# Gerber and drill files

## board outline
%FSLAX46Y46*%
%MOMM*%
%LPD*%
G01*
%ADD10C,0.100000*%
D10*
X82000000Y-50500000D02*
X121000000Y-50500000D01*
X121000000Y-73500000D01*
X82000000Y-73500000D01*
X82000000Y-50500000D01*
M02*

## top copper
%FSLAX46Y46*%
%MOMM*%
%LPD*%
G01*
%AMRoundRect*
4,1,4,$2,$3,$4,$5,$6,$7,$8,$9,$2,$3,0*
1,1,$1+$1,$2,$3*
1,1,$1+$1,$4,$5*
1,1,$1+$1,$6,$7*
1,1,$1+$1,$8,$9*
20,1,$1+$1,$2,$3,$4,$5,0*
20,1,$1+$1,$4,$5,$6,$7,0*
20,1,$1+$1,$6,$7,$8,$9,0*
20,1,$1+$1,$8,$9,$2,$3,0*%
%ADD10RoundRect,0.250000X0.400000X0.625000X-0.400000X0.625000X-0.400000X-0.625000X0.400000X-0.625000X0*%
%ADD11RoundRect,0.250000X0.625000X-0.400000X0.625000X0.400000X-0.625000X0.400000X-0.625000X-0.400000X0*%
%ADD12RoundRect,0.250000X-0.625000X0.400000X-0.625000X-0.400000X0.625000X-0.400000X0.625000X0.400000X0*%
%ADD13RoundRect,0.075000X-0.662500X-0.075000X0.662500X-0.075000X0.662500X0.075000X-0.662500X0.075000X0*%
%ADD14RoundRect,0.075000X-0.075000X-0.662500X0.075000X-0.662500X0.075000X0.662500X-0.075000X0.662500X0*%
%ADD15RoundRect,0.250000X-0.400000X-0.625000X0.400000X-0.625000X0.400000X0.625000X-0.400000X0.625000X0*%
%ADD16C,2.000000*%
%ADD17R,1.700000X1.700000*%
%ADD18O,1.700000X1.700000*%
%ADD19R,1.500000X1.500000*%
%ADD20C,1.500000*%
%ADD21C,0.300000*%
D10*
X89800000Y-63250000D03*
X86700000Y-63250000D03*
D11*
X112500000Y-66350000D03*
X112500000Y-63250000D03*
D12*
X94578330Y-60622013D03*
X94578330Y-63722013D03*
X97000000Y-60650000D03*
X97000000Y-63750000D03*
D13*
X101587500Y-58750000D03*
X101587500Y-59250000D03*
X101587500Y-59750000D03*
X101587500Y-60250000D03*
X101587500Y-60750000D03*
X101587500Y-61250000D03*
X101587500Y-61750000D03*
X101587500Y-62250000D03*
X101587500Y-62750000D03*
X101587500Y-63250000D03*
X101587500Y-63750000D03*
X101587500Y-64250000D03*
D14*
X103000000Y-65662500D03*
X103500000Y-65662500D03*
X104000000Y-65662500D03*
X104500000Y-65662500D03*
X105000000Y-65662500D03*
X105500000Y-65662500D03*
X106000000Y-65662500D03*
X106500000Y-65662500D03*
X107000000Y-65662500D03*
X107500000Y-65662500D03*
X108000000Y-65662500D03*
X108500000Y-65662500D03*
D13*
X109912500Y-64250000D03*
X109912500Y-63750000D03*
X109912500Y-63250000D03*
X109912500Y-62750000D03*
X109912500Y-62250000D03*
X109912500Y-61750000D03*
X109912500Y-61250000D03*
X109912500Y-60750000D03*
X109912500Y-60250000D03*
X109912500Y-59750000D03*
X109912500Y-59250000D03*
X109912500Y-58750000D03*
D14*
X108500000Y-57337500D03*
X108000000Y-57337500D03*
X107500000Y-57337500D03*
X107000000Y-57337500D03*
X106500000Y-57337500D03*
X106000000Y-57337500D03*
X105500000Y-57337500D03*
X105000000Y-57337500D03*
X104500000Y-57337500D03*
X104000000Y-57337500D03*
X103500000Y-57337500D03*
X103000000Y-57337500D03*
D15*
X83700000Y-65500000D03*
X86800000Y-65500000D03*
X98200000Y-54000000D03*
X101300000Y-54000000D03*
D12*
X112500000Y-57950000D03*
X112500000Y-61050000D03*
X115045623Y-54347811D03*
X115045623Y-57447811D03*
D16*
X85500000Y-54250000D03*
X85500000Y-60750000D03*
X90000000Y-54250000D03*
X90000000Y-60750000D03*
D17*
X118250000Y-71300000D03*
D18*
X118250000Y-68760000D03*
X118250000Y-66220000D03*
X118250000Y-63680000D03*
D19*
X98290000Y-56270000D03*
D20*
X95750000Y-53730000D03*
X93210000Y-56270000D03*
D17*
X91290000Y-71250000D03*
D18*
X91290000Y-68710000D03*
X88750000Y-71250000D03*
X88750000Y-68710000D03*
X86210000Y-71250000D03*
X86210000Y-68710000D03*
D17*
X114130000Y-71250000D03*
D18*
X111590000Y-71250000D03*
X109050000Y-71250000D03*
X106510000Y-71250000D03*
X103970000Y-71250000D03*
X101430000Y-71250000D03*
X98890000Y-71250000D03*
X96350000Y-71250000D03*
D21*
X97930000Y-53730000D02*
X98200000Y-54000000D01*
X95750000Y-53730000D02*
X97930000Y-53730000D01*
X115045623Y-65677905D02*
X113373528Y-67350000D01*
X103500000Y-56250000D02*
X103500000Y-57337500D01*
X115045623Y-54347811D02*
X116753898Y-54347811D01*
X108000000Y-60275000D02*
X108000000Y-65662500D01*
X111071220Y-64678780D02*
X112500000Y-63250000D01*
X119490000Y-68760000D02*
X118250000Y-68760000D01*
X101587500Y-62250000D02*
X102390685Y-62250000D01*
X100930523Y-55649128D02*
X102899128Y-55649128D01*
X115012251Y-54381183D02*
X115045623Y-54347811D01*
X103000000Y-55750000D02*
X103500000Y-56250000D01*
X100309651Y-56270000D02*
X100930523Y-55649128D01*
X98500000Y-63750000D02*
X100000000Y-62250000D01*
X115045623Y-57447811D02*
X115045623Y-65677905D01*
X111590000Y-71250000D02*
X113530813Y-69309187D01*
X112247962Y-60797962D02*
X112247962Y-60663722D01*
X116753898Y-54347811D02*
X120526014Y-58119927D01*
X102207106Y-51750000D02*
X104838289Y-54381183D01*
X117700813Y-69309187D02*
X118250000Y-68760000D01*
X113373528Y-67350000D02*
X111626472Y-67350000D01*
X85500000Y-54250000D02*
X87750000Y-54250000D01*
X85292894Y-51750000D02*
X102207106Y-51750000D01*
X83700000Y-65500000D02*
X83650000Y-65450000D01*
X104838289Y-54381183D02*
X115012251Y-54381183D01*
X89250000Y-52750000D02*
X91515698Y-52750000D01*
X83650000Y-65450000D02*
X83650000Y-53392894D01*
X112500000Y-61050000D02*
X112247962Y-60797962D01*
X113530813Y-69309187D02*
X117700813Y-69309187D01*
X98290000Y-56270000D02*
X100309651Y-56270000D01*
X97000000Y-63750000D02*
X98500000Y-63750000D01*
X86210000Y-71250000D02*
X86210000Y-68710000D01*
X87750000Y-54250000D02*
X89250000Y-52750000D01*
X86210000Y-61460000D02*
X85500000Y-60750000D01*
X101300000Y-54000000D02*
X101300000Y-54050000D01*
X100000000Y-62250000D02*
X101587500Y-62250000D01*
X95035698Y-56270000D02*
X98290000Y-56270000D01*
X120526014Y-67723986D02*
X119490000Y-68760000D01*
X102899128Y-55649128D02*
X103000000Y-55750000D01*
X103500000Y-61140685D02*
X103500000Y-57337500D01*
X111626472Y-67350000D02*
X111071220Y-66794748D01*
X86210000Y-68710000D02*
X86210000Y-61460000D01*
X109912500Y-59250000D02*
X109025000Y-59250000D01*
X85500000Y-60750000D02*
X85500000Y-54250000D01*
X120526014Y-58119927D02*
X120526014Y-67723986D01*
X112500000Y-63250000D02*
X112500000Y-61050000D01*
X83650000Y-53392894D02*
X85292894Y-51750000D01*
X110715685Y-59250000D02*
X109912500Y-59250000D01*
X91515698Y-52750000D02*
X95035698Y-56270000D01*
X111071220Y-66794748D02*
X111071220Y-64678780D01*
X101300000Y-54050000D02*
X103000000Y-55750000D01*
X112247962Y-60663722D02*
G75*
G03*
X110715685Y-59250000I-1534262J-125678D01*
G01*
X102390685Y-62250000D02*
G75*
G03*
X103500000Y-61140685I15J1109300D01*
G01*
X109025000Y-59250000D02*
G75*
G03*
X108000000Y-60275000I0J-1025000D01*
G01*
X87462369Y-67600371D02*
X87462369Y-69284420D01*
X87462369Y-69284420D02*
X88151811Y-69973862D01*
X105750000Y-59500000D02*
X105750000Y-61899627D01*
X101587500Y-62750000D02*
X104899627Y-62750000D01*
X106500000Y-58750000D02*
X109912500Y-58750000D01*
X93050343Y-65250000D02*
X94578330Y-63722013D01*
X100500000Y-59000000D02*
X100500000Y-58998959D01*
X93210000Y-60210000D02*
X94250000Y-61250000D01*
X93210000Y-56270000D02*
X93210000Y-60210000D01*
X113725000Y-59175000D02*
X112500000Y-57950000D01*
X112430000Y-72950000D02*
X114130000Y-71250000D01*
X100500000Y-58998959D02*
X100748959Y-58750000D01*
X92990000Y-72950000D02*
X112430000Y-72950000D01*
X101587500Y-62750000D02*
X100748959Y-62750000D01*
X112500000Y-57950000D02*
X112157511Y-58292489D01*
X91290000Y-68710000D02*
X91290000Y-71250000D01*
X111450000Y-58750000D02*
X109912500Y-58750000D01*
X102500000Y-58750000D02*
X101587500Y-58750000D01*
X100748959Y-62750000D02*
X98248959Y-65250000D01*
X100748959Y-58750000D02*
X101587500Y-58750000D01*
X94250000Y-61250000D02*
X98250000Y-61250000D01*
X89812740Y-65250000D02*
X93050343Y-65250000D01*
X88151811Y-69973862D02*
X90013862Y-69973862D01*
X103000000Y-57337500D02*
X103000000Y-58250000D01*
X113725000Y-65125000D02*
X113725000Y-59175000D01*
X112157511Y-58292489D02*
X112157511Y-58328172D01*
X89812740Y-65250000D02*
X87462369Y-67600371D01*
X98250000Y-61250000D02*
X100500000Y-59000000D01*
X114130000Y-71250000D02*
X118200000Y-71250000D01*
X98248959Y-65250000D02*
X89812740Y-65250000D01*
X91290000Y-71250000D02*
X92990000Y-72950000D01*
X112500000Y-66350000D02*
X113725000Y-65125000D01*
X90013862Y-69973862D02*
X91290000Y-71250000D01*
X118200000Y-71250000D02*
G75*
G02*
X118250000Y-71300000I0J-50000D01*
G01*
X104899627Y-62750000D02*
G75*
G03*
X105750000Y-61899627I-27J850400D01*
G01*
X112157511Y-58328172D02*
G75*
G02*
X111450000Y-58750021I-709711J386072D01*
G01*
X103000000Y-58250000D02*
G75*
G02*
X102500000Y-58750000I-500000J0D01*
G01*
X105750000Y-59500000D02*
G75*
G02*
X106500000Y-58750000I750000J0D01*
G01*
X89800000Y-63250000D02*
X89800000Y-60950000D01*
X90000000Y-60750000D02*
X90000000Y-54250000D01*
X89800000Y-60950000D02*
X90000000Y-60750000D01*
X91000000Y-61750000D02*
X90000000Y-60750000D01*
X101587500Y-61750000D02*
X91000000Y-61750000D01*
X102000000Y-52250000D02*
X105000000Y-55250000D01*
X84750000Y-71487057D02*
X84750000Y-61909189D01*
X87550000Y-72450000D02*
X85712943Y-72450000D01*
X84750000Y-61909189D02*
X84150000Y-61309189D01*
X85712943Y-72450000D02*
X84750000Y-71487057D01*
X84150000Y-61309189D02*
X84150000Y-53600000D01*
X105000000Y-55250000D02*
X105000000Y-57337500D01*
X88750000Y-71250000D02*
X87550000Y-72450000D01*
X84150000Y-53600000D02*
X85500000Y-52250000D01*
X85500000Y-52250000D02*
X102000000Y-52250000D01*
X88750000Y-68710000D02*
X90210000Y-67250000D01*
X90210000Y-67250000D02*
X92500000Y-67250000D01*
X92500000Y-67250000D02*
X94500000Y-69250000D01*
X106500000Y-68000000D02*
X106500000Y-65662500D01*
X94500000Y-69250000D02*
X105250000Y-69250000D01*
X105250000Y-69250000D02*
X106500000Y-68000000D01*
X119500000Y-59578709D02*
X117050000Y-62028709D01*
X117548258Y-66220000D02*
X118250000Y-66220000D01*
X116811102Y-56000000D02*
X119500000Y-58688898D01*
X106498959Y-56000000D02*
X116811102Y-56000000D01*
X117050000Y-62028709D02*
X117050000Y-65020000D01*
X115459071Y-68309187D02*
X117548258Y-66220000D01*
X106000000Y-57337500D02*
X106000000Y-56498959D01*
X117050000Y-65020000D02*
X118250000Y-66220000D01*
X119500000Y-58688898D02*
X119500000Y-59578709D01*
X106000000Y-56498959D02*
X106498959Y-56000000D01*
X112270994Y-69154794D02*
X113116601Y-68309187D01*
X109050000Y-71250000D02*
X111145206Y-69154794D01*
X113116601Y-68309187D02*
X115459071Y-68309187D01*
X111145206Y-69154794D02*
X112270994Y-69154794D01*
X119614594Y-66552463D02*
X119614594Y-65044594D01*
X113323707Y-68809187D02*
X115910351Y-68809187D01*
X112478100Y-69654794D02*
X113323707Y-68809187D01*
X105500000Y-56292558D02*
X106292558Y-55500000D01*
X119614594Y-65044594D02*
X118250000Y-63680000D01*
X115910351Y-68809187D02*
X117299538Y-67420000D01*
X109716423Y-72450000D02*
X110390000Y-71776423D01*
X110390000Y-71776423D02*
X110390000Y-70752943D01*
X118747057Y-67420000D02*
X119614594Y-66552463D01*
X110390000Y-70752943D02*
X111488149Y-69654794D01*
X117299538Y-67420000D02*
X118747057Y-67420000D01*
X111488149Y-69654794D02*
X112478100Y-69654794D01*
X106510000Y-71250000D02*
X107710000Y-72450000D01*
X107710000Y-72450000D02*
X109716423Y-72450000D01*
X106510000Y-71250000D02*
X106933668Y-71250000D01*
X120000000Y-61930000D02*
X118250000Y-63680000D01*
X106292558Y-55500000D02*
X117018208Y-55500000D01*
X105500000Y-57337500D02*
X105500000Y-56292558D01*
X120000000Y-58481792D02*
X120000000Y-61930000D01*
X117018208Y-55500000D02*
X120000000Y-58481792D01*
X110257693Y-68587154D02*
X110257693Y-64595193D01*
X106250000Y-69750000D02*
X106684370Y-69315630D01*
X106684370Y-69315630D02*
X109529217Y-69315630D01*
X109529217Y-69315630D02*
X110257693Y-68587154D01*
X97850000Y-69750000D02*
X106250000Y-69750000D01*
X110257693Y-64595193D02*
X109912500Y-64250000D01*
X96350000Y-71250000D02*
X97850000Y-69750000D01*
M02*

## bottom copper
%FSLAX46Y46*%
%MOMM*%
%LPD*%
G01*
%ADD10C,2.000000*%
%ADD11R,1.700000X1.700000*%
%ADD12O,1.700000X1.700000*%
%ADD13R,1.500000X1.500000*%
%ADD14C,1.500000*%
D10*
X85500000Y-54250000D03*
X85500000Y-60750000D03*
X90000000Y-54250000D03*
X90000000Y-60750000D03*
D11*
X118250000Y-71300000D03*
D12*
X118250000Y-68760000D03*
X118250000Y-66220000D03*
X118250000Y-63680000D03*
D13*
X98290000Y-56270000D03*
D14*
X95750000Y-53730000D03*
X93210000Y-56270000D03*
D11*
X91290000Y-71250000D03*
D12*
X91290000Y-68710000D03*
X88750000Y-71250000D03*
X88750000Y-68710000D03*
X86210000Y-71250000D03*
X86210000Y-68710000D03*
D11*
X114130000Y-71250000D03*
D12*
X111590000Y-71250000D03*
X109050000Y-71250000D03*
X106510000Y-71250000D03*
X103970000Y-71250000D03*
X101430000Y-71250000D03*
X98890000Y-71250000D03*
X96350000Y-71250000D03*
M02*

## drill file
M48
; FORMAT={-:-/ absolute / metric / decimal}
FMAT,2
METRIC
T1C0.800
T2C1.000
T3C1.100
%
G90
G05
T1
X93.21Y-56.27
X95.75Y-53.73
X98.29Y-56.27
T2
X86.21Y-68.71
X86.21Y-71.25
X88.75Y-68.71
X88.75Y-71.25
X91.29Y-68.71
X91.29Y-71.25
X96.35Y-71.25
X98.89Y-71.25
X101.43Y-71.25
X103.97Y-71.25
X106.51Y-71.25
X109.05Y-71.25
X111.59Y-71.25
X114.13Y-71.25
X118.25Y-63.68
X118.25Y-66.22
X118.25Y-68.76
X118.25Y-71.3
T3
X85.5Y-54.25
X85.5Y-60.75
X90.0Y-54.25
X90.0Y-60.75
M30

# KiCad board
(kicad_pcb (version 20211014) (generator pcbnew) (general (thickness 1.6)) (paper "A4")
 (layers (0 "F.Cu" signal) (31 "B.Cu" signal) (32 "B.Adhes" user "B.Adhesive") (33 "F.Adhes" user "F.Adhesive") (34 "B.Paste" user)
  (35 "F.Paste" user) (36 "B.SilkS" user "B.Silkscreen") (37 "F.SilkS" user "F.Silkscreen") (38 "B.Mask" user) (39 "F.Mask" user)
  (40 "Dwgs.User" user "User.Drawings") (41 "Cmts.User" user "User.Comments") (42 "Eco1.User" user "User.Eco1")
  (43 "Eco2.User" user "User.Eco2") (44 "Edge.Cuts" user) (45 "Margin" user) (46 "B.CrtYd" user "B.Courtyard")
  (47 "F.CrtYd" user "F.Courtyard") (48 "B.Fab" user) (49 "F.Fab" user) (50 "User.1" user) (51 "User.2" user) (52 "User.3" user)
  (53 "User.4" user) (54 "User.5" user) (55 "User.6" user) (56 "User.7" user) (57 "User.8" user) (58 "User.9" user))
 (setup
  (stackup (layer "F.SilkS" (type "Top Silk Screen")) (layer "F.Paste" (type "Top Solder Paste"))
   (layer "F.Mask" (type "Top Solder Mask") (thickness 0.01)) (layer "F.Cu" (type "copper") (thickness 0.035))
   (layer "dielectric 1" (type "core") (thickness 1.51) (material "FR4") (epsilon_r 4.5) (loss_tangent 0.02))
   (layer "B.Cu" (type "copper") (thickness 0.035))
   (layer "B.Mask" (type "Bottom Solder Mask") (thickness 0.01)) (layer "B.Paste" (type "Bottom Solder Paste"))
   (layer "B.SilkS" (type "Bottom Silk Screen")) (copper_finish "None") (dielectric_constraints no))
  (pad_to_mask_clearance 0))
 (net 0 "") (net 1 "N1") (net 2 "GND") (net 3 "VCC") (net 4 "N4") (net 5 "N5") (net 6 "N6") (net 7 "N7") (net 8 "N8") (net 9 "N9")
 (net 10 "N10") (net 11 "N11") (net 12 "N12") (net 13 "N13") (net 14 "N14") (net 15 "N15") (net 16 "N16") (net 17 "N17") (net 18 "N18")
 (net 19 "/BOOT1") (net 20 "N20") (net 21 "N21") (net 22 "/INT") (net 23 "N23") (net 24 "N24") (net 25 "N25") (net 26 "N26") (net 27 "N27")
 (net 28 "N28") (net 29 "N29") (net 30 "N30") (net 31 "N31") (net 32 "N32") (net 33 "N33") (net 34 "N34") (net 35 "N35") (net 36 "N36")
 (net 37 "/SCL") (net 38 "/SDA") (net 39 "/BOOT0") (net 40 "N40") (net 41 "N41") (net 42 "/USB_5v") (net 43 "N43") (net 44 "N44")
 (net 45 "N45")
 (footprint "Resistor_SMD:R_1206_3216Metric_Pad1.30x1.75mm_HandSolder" (layer "F.Cu") (at 88.25 63.25 180)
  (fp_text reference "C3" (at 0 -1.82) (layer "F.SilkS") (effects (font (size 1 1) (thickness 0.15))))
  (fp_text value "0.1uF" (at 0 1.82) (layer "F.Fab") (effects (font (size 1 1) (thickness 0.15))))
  (pad "1" smd roundrect (at -1.55 0 180) (size 1.3 1.75) (layers "F.Cu" "F.Paste" "F.Mask") (roundrect_rratio 0.1923076923) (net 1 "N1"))
  (pad "2" smd roundrect (at 1.55 0 180) (size 1.3 1.75) (layers "F.Cu" "F.Paste" "F.Mask") (roundrect_rratio 0.1923076923) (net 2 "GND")))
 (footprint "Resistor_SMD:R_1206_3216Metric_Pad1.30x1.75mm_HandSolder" (layer "F.Cu") (at 112.5 64.8 90)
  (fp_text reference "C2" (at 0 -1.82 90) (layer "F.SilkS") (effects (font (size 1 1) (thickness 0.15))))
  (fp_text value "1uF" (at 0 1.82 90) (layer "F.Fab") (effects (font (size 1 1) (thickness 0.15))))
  (pad "1" smd roundrect (at -1.55 0 90) (size 1.3 1.75) (layers "F.Cu" "F.Paste" "F.Mask") (roundrect_rratio 0.1923076923) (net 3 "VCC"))
  (pad "2" smd roundrect (at 1.55 0 90) (size 1.3 1.75) (layers "F.Cu" "F.Paste" "F.Mask") (roundrect_rratio 0.1923076923) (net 2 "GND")))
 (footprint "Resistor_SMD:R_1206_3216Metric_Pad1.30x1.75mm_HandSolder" (layer "F.Cu") (at 94.57833 62.172013 -90)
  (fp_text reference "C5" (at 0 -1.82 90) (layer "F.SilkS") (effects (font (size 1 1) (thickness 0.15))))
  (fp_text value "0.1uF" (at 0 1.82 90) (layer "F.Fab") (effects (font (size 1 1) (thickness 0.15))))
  (pad "1" smd roundrect (at -1.55 0 270) (size 1.3 1.75) (layers "F.Cu" "F.Paste" "F.Mask") (roundrect_rratio 0.1923076923) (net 3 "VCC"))
  (pad "2" smd roundrect (at 1.55 0 270) (size 1.3 1.75) (layers "F.Cu" "F.Paste" "F.Mask") (roundrect_rratio 0.1923076923) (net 3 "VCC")))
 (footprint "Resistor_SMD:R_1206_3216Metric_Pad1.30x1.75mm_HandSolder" (layer "F.Cu") (at 97 62.2 -90)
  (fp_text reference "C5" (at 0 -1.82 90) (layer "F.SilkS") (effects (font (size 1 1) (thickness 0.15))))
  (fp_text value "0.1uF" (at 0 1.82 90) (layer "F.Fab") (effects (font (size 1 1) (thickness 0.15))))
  (pad "1" smd roundrect (at -1.55 0 270) (size 1.3 1.75) (layers "F.Cu" "F.Paste" "F.Mask") (roundrect_rratio 0.1923076923) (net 3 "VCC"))
  (pad "2" smd roundrect (at 1.55 0 270) (size 1.3 1.75) (layers "F.Cu" "F.Paste" "F.Mask") (roundrect_rratio 0.1923076923) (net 2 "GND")))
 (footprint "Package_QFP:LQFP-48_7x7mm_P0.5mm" (layer "F.Cu") (at 105.75 61.5)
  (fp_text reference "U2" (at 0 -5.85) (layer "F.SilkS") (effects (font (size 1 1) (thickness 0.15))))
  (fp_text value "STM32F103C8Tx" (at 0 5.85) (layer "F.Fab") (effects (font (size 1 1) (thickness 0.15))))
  (pad "1" smd roundrect (at -4.1625 -2.75) (size 1.475 0.3) (layers "F.Cu" "F.Paste" "F.Mask") (roundrect_rratio 0.25) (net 3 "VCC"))
  (pad "2" smd roundrect (at -4.1625 -2.25) (size 1.475 0.3) (layers "F.Cu" "F.Paste" "F.Mask") (roundrect_rratio 0.25) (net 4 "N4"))
  (pad "3" smd roundrect (at -4.1625 -1.75) (size 1.475 0.3) (layers "F.Cu" "F.Paste" "F.Mask") (roundrect_rratio 0.25) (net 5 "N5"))
  (pad "4" smd roundrect (at -4.1625 -1.25) (size 1.475 0.3) (layers "F.Cu" "F.Paste" "F.Mask") (roundrect_rratio 0.25) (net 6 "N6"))
  (pad "5" smd roundrect (at -4.1625 -0.75) (size 1.475 0.3) (layers "F.Cu" "F.Paste" "F.Mask") (roundrect_rratio 0.25) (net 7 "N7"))
  (pad "6" smd roundrect (at -4.1625 -0.25) (size 1.475 0.3) (layers "F.Cu" "F.Paste" "F.Mask") (roundrect_rratio 0.25) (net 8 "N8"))
  (pad "7" smd roundrect (at -4.1625 0.25) (size 1.475 0.3) (layers "F.Cu" "F.Paste" "F.Mask") (roundrect_rratio 0.25) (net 1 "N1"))
  (pad "8" smd roundrect (at -4.1625 0.75) (size 1.475 0.3) (layers "F.Cu" "F.Paste" "F.Mask") (roundrect_rratio 0.25) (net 2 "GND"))
  (pad "9" smd roundrect (at -4.1625 1.25) (size 1.475 0.3) (layers "F.Cu" "F.Paste" "F.Mask") (roundrect_rratio 0.25) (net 3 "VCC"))
  (pad "10" smd roundrect (at -4.1625 1.75) (size 1.475 0.3) (layers "F.Cu" "F.Paste" "F.Mask") (roundrect_rratio 0.25) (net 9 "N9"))
  (pad "11" smd roundrect (at -4.1625 2.25) (size 1.475 0.3) (layers "F.Cu" "F.Paste" "F.Mask") (roundrect_rratio 0.25) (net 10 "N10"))
  (pad "12" smd roundrect (at -4.1625 2.75) (size 1.475 0.3) (layers "F.Cu" "F.Paste" "F.Mask") (roundrect_rratio 0.25) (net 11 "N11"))
  (pad "13" smd roundrect (at -2.75 4.1625) (size 0.3 1.475) (layers "F.Cu" "F.Paste" "F.Mask") (roundrect_rratio 0.25) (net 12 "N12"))
  (pad "14" smd roundrect (at -2.25 4.1625) (size 0.3 1.475) (layers "F.Cu" "F.Paste" "F.Mask") (roundrect_rratio 0.25) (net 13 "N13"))
  (pad "15" smd roundrect (at -1.75 4.1625) (size 0.3 1.475) (layers "F.Cu" "F.Paste" "F.Mask") (roundrect_rratio 0.25) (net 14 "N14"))
  (pad "16" smd roundrect (at -1.25 4.1625) (size 0.3 1.475) (layers "F.Cu" "F.Paste" "F.Mask") (roundrect_rratio 0.25) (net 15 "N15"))
  (pad "17" smd roundrect (at -0.75 4.1625) (size 0.3 1.475) (layers "F.Cu" "F.Paste" "F.Mask") (roundrect_rratio 0.25) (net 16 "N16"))
  (pad "18" smd roundrect (at -0.25 4.1625) (size 0.3 1.475) (layers "F.Cu" "F.Paste" "F.Mask") (roundrect_rratio 0.25) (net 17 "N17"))
  (pad "19" smd roundrect (at 0.25 4.1625) (size 0.3 1.475) (layers "F.Cu" "F.Paste" "F.Mask") (roundrect_rratio 0.25) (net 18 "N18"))
  (pad "20" smd roundrect (at 0.75 4.1625) (size 0.3 1.475) (layers "F.Cu" "F.Paste" "F.Mask") (roundrect_rratio 0.25) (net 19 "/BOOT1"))
  (pad "21" smd roundrect (at 1.25 4.1625) (size 0.3 1.475) (layers "F.Cu" "F.Paste" "F.Mask") (roundrect_rratio 0.25) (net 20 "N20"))
  (pad "22" smd roundrect (at 1.75 4.1625) (size 0.3 1.475) (layers "F.Cu" "F.Paste" "F.Mask") (roundrect_rratio 0.25) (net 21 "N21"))
  (pad "23" smd roundrect (at 2.25 4.1625) (size 0.3 1.475) (layers "F.Cu" "F.Paste" "F.Mask") (roundrect_rratio 0.25) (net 2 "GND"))
  (pad "24" smd roundrect (at 2.75 4.1625) (size 0.3 1.475) (layers "F.Cu" "F.Paste" "F.Mask") (roundrect_rratio 0.25) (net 3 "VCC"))
  (pad "25" smd roundrect (at 4.1625 2.75) (size 1.475 0.3) (layers "F.Cu" "F.Paste" "F.Mask") (roundrect_rratio 0.25) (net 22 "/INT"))
  (pad "26" smd roundrect (at 4.1625 2.25) (size 1.475 0.3) (layers "F.Cu" "F.Paste" "F.Mask") (roundrect_rratio 0.25) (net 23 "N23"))
  (pad "27" smd roundrect (at 4.1625 1.75) (size 1.475 0.3) (layers "F.Cu" "F.Paste" "F.Mask") (roundrect_rratio 0.25) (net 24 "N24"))
  (pad "28" smd roundrect (at 4.1625 1.25) (size 1.475 0.3) (layers "F.Cu" "F.Paste" "F.Mask") (roundrect_rratio 0.25) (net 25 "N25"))
  (pad "29" smd roundrect (at 4.1625 0.75) (size 1.475 0.3) (layers "F.Cu" "F.Paste" "F.Mask") (roundrect_rratio 0.25) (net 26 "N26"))
  (pad "30" smd roundrect (at 4.1625 0.25) (size 1.475 0.3) (layers "F.Cu" "F.Paste" "F.Mask") (roundrect_rratio 0.25) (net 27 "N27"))
  (pad "31" smd roundrect (at 4.1625 -0.25) (size 1.475 0.3) (layers "F.Cu" "F.Paste" "F.Mask") (roundrect_rratio 0.25) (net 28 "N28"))
  (pad "32" smd roundrect (at 4.1625 -0.75) (size 1.475 0.3) (layers "F.Cu" "F.Paste" "F.Mask") (roundrect_rratio 0.25) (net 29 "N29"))
  (pad "33" smd roundrect (at 4.1625 -1.25) (size 1.475 0.3) (layers "F.Cu" "F.Paste" "F.Mask") (roundrect_rratio 0.25) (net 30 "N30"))
  (pad "34" smd roundrect (at 4.1625 -1.75) (size 1.475 0.3) (layers "F.Cu" "F.Paste" "F.Mask") (roundrect_rratio 0.25) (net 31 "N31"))
  (pad "35" smd roundrect (at 4.1625 -2.25) (size 1.475 0.3) (layers "F.Cu" "F.Paste" "F.Mask") (roundrect_rratio 0.25) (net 2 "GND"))
  (pad "36" smd roundrect (at 4.1625 -2.75) (size 1.475 0.3) (layers "F.Cu" "F.Paste" "F.Mask") (roundrect_rratio 0.25) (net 3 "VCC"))
  (pad "37" smd roundrect (at 2.75 -4.1625) (size 0.3 1.475) (layers "F.Cu" "F.Paste" "F.Mask") (roundrect_rratio 0.25) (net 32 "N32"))
  (pad "38" smd roundrect (at 2.25 -4.1625) (size 0.3 1.475) (layers "F.Cu" "F.Paste" "F.Mask") (roundrect_rratio 0.25) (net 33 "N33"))
  (pad "39" smd roundrect (at 1.75 -4.1625) (size 0.3 1.475) (layers "F.Cu" "F.Paste" "F.Mask") (roundrect_rratio 0.25) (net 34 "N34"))
  (pad "40" smd roundrect (at 1.25 -4.1625) (size 0.3 1.475) (layers "F.Cu" "F.Paste" "F.Mask") (roundrect_rratio 0.25) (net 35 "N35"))
  (pad "41" smd roundrect (at 0.75 -4.1625) (size 0.3 1.475) (layers "F.Cu" "F.Paste" "F.Mask") (roundrect_rratio 0.25) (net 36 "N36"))
  (pad "42" smd roundrect (at 0.25 -4.1625) (size 0.3 1.475) (layers "F.Cu" "F.Paste" "F.Mask") (roundrect_rratio 0.25) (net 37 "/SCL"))
  (pad "43" smd roundrect (at -0.25 -4.1625) (size 0.3 1.475) (layers "F.Cu" "F.Paste" "F.Mask") (roundrect_rratio 0.25) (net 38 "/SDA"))
  (pad "44" smd roundrect (at -0.75 -4.1625) (size 0.3 1.475) (layers "F.Cu" "F.Paste" "F.Mask") (roundrect_rratio 0.25) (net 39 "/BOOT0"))
  (pad "45" smd roundrect (at -1.25 -4.1625) (size 0.3 1.475) (layers "F.Cu" "F.Paste" "F.Mask") (roundrect_rratio 0.25) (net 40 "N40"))
  (pad "46" smd roundrect (at -1.75 -4.1625) (size 0.3 1.475) (layers "F.Cu" "F.Paste" "F.Mask") (roundrect_rratio 0.25) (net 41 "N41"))
  (pad "47" smd roundrect (at -2.25 -4.1625) (size 0.3 1.475) (layers "F.Cu" "F.Paste" "F.Mask") (roundrect_rratio 0.25) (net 2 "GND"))
  (pad "48" smd roundrect (at -2.75 -4.1625) (size 0.3 1.475) (layers "F.Cu" "F.Paste" "F.Mask") (roundrect_rratio 0.25) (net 3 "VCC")))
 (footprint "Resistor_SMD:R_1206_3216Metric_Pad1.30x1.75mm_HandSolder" (layer "F.Cu") (at 85.25 65.5)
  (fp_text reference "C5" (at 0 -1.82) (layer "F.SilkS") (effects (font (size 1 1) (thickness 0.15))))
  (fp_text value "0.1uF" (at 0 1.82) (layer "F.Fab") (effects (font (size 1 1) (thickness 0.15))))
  (pad "1" smd roundrect (at -1.55 0) (size 1.3 1.75) (layers "F.Cu" "F.Paste" "F.Mask") (roundrect_rratio 0.1923076923) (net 2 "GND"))
  (pad "2" smd roundrect (at 1.55 0) (size 1.3 1.75) (layers "F.Cu" "F.Paste" "F.Mask") (roundrect_rratio 0.1923076923) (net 2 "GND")))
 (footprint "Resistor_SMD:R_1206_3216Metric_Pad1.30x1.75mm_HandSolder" (layer "F.Cu") (at 99.75 54)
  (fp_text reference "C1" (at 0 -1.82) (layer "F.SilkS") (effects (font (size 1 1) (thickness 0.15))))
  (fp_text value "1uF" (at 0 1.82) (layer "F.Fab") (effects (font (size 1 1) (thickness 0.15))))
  (pad "1" smd roundrect (at -1.55 0) (size 1.3 1.75) (layers "F.Cu" "F.Paste" "F.Mask") (roundrect_rratio 0.1923076923) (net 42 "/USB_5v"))
  (pad "2" smd roundrect (at 1.55 0) (size 1.3 1.75) (layers "F.Cu" "F.Paste" "F.Mask") (roundrect_rratio 0.1923076923) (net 2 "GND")))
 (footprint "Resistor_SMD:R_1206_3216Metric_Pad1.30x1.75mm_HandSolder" (layer "F.Cu") (at 112.5 59.5 -90)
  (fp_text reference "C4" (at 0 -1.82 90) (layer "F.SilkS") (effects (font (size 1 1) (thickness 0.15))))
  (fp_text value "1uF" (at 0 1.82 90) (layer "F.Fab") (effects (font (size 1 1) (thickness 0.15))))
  (pad "1" smd roundrect (at -1.55 0 270) (size 1.3 1.75) (layers "F.Cu" "F.Paste" "F.Mask") (roundrect_rratio 0.1923076923) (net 3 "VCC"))
  (pad "2" smd roundrect (at 1.55 0 270) (size 1.3 1.75) (layers "F.Cu" "F.Paste" "F.Mask") (roundrect_rratio 0.1923076923) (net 2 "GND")))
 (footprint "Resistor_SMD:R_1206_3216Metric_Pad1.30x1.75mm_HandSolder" (layer "F.Cu") (at 115.045623 55.897811 -90)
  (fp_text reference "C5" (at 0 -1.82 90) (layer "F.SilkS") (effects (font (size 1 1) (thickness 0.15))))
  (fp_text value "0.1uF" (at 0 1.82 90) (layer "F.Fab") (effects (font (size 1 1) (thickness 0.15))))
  (pad "1" smd roundrect (at -1.55 0 270) (size 1.3 1.75) (layers "F.Cu" "F.Paste" "F.Mask") (roundrect_rratio 0.1923076923) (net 2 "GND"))
  (pad "2" smd roundrect (at 1.55 0 270) (size 1.3 1.75) (layers "F.Cu" "F.Paste" "F.Mask") (roundrect_rratio 0.1923076923) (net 2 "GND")))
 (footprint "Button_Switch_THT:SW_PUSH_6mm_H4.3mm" (layer "B.Cu") (at 85.5 54.25 -90)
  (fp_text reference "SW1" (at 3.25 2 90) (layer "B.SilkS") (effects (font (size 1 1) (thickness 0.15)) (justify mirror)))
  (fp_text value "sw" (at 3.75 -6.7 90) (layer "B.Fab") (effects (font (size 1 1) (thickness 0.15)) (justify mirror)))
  (pad "1" thru_hole circle (at 0 0 180) (size 2 2) (drill 1.1) (layers *.Cu *.Mask) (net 2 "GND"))
  (pad "1" thru_hole circle (at 6.5 0 180) (size 2 2) (drill 1.1) (layers *.Cu *.Mask) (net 2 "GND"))
  (pad "2" thru_hole circle (at 0 -4.5 180) (size 2 2) (drill 1.1) (layers *.Cu *.Mask) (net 1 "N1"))
  (pad "2" thru_hole circle (at 6.5 -4.5 180) (size 2 2) (drill 1.1) (layers *.Cu *.Mask) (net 1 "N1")))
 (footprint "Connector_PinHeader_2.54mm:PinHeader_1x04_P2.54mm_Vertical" (layer "B.Cu") (at 118.25 71.3)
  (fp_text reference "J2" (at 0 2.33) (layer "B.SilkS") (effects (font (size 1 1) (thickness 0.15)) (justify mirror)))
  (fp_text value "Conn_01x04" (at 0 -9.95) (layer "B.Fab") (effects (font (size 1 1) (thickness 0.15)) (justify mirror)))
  (pad "1" thru_hole rect (at 0 0) (size 1.7 1.7) (drill 1) (layers *.Cu *.Mask) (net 3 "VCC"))
  (pad "2" thru_hole oval (at 0 -2.54) (size 1.7 1.7) (drill 1) (layers *.Cu *.Mask) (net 2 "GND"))
  (pad "3" thru_hole oval (at 0 -5.08) (size 1.7 1.7) (drill 1) (layers *.Cu *.Mask) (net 37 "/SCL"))
  (pad "4" thru_hole oval (at 0 -7.62) (size 1.7 1.7) (drill 1) (layers *.Cu *.Mask) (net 38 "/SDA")))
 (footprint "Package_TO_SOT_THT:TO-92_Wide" (layer "B.Cu") (at 98.29 56.27 180)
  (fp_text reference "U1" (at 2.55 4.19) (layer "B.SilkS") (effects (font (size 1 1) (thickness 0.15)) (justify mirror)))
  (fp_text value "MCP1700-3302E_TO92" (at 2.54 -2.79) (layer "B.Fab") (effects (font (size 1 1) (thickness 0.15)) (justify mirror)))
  (pad "1" thru_hole rect (at 0 0 180) (size 1.5 1.5) (drill 0.8) (layers *.Cu *.Mask) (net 2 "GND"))
  (pad "2" thru_hole circle (at 2.54 2.54 180) (size 1.5 1.5) (drill 0.8) (layers *.Cu *.Mask) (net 42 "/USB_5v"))
  (pad "3" thru_hole circle (at 5.08 0 180) (size 1.5 1.5) (drill 0.8) (layers *.Cu *.Mask) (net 3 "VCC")))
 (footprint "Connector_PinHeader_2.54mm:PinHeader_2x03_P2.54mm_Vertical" (layer "B.Cu") (at 91.29 71.25 90)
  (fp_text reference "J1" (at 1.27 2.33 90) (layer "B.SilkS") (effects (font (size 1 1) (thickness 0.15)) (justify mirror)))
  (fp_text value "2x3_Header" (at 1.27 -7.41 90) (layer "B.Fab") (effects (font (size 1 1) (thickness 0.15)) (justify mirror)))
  (pad "1" thru_hole rect (at 0 0 90) (size 1.7 1.7) (drill 1) (layers *.Cu *.Mask) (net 3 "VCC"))
  (pad "2" thru_hole oval (at 2.54 0 90) (size 1.7 1.7) (drill 1) (layers *.Cu *.Mask) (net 3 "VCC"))
  (pad "3" thru_hole oval (at 0 -2.54 90) (size 1.7 1.7) (drill 1) (layers *.Cu *.Mask) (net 39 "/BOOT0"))
  (pad "4" thru_hole oval (at 2.54 -2.54 90) (size 1.7 1.7) (drill 1) (layers *.Cu *.Mask) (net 19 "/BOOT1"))
  (pad "5" thru_hole oval (at 0 -5.08 90) (size 1.7 1.7) (drill 1) (layers *.Cu *.Mask) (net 2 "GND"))
  (pad "6" thru_hole oval (at 2.54 -5.08 90) (size 1.7 1.7) (drill 1) (layers *.Cu *.Mask) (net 2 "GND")))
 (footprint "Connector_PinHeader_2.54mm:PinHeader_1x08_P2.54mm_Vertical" (layer "B.Cu") (at 114.13 71.25 90)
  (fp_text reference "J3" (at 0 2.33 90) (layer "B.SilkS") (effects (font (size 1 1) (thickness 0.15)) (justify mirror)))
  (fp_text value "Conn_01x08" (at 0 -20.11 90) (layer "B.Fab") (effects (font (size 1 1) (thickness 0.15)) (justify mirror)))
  (pad "1" thru_hole rect (at 0 0 90) (size 1.7 1.7) (drill 1) (layers *.Cu *.Mask) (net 3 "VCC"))
  (pad "2" thru_hole oval (at 0 -2.54 90) (size 1.7 1.7) (drill 1) (layers *.Cu *.Mask) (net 2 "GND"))
  (pad "3" thru_hole oval (at 0 -5.08 90) (size 1.7 1.7) (drill 1) (layers *.Cu *.Mask) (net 37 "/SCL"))
  (pad "4" thru_hole oval (at 0 -7.62 90) (size 1.7 1.7) (drill 1) (layers *.Cu *.Mask) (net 38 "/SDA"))
  (pad "5" thru_hole oval (at 0 -10.16 90) (size 1.7 1.7) (drill 1) (layers *.Cu *.Mask) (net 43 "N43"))
  (pad "6" thru_hole oval (at 0 -12.7 90) (size 1.7 1.7) (drill 1) (layers *.Cu *.Mask) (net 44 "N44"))
  (pad "7" thru_hole oval (at 0 -15.24 90) (size 1.7 1.7) (drill 1) (layers *.Cu *.Mask) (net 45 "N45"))
  (pad "8" thru_hole oval (at 0 -17.78 90) (size 1.7 1.7) (drill 1) (layers *.Cu *.Mask) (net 22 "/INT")))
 (gr_rect (start 121 73.5) (end 82 50.5) (layer "Edge.Cuts") (width 0.1) (fill none))
 (segment (start 97.93 53.73) (end 98.2 54) (width 0.3) (layer "F.Cu") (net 42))
 (segment (start 95.75 53.73) (end 97.93 53.73) (width 0.3) (layer "F.Cu") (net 42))
 (segment (start 115.045623 65.677905) (end 113.373528 67.35) (width 0.3) (layer "F.Cu") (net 2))
 (segment (start 103.5 56.25) (end 103.5 57.3375) (width 0.3) (layer "F.Cu") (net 2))
 (segment (start 115.045623 54.347811) (end 116.753898 54.347811) (width 0.3) (layer "F.Cu") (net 2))
 (segment (start 108 60.275) (end 108 65.6625) (width 0.3) (layer "F.Cu") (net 2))
 (segment (start 111.07122 64.67878) (end 112.5 63.25) (width 0.3) (layer "F.Cu") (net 2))
 (segment (start 119.49 68.76) (end 118.25 68.76) (width 0.3) (layer "F.Cu") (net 2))
 (segment (start 101.5875 62.25) (end 102.390685 62.25) (width 0.3) (layer "F.Cu") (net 2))
 (segment (start 100.930523 55.649128) (end 102.899128 55.649128) (width 0.3) (layer "F.Cu") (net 2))
 (segment (start 115.012251 54.381183) (end 115.045623 54.347811) (width 0.3) (layer "F.Cu") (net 2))
 (segment (start 103 55.75) (end 103.5 56.25) (width 0.3) (layer "F.Cu") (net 2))
 (segment (start 100.309651 56.27) (end 100.930523 55.649128) (width 0.3) (layer "F.Cu") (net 2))
 (segment (start 98.5 63.75) (end 100 62.25) (width 0.3) (layer "F.Cu") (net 2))
 (segment (start 115.045623 57.447811) (end 115.045623 65.677905) (width 0.3) (layer "F.Cu") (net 2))
 (segment (start 111.59 71.25) (end 113.530813 69.309187) (width 0.3) (layer "F.Cu") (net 2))
 (segment (start 112.247962 60.797962) (end 112.247962 60.663722) (width 0.3) (layer "F.Cu") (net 2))
 (segment (start 116.753898 54.347811) (end 120.526014 58.119927) (width 0.3) (layer "F.Cu") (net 2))
 (segment (start 102.207106 51.75) (end 104.838289 54.381183) (width 0.3) (layer "F.Cu") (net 2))
 (segment (start 117.700813 69.309187) (end 118.25 68.76) (width 0.3) (layer "F.Cu") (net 2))
 (segment (start 113.373528 67.35) (end 111.626472 67.35) (width 0.3) (layer "F.Cu") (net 2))
 (segment (start 85.5 54.25) (end 87.75 54.25) (width 0.3) (layer "F.Cu") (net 2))
 (segment (start 85.292894 51.75) (end 102.207106 51.75) (width 0.3) (layer "F.Cu") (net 2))
 (segment (start 83.7 65.5) (end 83.65 65.45) (width 0.3) (layer "F.Cu") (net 2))
 (segment (start 104.838289 54.381183) (end 115.012251 54.381183) (width 0.3) (layer "F.Cu") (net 2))
 (segment (start 89.25 52.75) (end 91.515698 52.75) (width 0.3) (layer "F.Cu") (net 2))
 (segment (start 83.65 65.45) (end 83.65 53.392894) (width 0.3) (layer "F.Cu") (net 2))
 (segment (start 112.5 61.05) (end 112.247962 60.797962) (width 0.3) (layer "F.Cu") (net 2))
 (segment (start 113.530813 69.309187) (end 117.700813 69.309187) (width 0.3) (layer "F.Cu") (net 2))
 (segment (start 98.29 56.27) (end 100.309651 56.27) (width 0.3) (layer "F.Cu") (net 2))
 (segment (start 97 63.75) (end 98.5 63.75) (width 0.3) (layer "F.Cu") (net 2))
 (segment (start 86.21 71.25) (end 86.21 68.71) (width 0.3) (layer "F.Cu") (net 2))
 (segment (start 87.75 54.25) (end 89.25 52.75) (width 0.3) (layer "F.Cu") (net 2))
 (segment (start 86.21 61.46) (end 85.5 60.75) (width 0.3) (layer "F.Cu") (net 2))
 (segment (start 101.3 54) (end 101.3 54.05) (width 0.3) (layer "F.Cu") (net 2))
 (segment (start 100 62.25) (end 101.5875 62.25) (width 0.3) (layer "F.Cu") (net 2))
 (segment (start 95.035698 56.27) (end 98.29 56.27) (width 0.3) (layer "F.Cu") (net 2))
 (segment (start 120.526014 67.723986) (end 119.49 68.76) (width 0.3) (layer "F.Cu") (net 2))
 (segment (start 102.899128 55.649128) (end 103 55.75) (width 0.3) (layer "F.Cu") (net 2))
 (segment (start 103.5 61.140685) (end 103.5 57.3375) (width 0.3) (layer "F.Cu") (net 2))
 (segment (start 111.626472 67.35) (end 111.07122 66.794748) (width 0.3) (layer "F.Cu") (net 2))
 (segment (start 86.21 68.71) (end 86.21 61.46) (width 0.3) (layer "F.Cu") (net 2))
 (segment (start 109.9125 59.25) (end 109.025 59.25) (width 0.3) (layer "F.Cu") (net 2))
 (segment (start 85.5 60.75) (end 85.5 54.25) (width 0.3) (layer "F.Cu") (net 2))
 (segment (start 120.526014 58.119927) (end 120.526014 67.723986) (width 0.3) (layer "F.Cu") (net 2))
 (segment (start 112.5 63.25) (end 112.5 61.05) (width 0.3) (layer "F.Cu") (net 2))
 (segment (start 83.65 53.392894) (end 85.292894 51.75) (width 0.3) (layer "F.Cu") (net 2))
 (segment (start 110.715685 59.25) (end 109.9125 59.25) (width 0.3) (layer "F.Cu") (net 2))
 (segment (start 91.515698 52.75) (end 95.035698 56.27) (width 0.3) (layer "F.Cu") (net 2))
 (segment (start 111.07122 66.794748) (end 111.07122 64.67878) (width 0.3) (layer "F.Cu") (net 2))
 (segment (start 101.3 54.05) (end 103 55.75) (width 0.3) (layer "F.Cu") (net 2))
 (arc (start 112.247962 60.663722) (mid 111.757183 59.657628) (end 110.715685 59.25) (width 0.3) (layer "F.Cu") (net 2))
 (arc (start 102.390685 62.25) (mid 103.175089 61.925089) (end 103.5 61.140685) (width 0.3) (layer "F.Cu") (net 2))
 (arc (start 109.025 59.25) (mid 108.300216 59.550216) (end 108 60.275) (width 0.3) (layer "F.Cu") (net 2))
 (segment (start 87.462369 67.600371) (end 87.462369 69.28442) (width 0.3) (layer "F.Cu") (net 3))
 (segment (start 87.462369 69.28442) (end 88.151811 69.973862) (width 0.3) (layer "F.Cu") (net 3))
 (segment (start 105.75 59.5) (end 105.75 61.899627) (width 0.3) (layer "F.Cu") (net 3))
 (segment (start 101.5875 62.75) (end 104.899627 62.75) (width 0.3) (layer "F.Cu") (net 3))
 (segment (start 106.5 58.75) (end 109.9125 58.75) (width 0.3) (layer "F.Cu") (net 3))
 (segment (start 93.050343 65.25) (end 94.57833 63.722013) (width 0.3) (layer "F.Cu") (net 3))
 (segment (start 100.5 59) (end 100.5 58.998959) (width 0.3) (layer "F.Cu") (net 3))
 (segment (start 93.21 60.21) (end 94.25 61.25) (width 0.3) (layer "F.Cu") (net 3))
 (segment (start 93.21 56.27) (end 93.21 60.21) (width 0.3) (layer "F.Cu") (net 3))
 (segment (start 113.725 59.175) (end 112.5 57.95) (width 0.3) (layer "F.Cu") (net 3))
 (segment (start 112.43 72.95) (end 114.13 71.25) (width 0.3) (layer "F.Cu") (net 3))
 (segment (start 100.5 58.998959) (end 100.748959 58.75) (width 0.3) (layer "F.Cu") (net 3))
 (segment (start 92.99 72.95) (end 112.43 72.95) (width 0.3) (layer "F.Cu") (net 3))
 (segment (start 101.5875 62.75) (end 100.748959 62.75) (width 0.3) (layer "F.Cu") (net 3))
 (segment (start 112.5 57.95) (end 112.157511 58.292489) (width 0.3) (layer "F.Cu") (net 3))
 (segment (start 91.29 68.71) (end 91.29 71.25) (width 0.3) (layer "F.Cu") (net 3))
 (segment (start 111.45 58.75) (end 109.9125 58.75) (width 0.3) (layer "F.Cu") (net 3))
 (segment (start 102.5 58.75) (end 101.5875 58.75) (width 0.3) (layer "F.Cu") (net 3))
 (segment (start 100.748959 62.75) (end 98.248959 65.25) (width 0.3) (layer "F.Cu") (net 3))
 (segment (start 100.748959 58.75) (end 101.5875 58.75) (width 0.3) (layer "F.Cu") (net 3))
 (segment (start 94.25 61.25) (end 98.25 61.25) (width 0.3) (layer "F.Cu") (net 3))
 (segment (start 89.81274 65.25) (end 93.050343 65.25) (width 0.3) (layer "F.Cu") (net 3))
 (segment (start 88.151811 69.973862) (end 90.013862 69.973862) (width 0.3) (layer "F.Cu") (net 3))
 (segment (start 103 57.3375) (end 103 58.25) (width 0.3) (layer "F.Cu") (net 3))
 (segment (start 113.725 65.125) (end 113.725 59.175) (width 0.3) (layer "F.Cu") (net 3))
 (segment (start 112.157511 58.292489) (end 112.157511 58.328172) (width 0.3) (layer "F.Cu") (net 3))
 (segment (start 89.81274 65.25) (end 87.462369 67.600371) (width 0.3) (layer "F.Cu") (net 3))
 (segment (start 98.25 61.25) (end 100.5 59) (width 0.3) (layer "F.Cu") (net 3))
 (segment (start 114.13 71.25) (end 118.2 71.25) (width 0.3) (layer "F.Cu") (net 3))
 (segment (start 98.248959 65.25) (end 89.81274 65.25) (width 0.3) (layer "F.Cu") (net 3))
 (segment (start 91.29 71.25) (end 92.99 72.95) (width 0.3) (layer "F.Cu") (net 3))
 (segment (start 112.5 66.35) (end 113.725 65.125) (width 0.3) (layer "F.Cu") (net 3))
 (segment (start 90.013862 69.973862) (end 91.29 71.25) (width 0.3) (layer "F.Cu") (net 3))
 (arc (start 118.2 71.25) (mid 118.235355 71.264645) (end 118.25 71.3) (width 0.3) (layer "F.Cu") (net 3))
 (arc (start 104.899627 62.75) (mid 105.500932 62.500932) (end 105.75 61.899627) (width 0.3) (layer "F.Cu") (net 3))
 (arc (start 112.157511 58.328172) (mid 111.861282 58.636183) (end 111.45 58.75) (width 0.3) (layer "F.Cu") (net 3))
 (arc (start 103 58.25) (mid 102.853553 58.603553) (end 102.5 58.75) (width 0.3) (layer "F.Cu") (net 3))
 (arc (start 105.75 59.5) (mid 105.96967 58.96967) (end 106.5 58.75) (width 0.3) (layer "F.Cu") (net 3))
 (segment (start 89.8 63.25) (end 89.8 60.95) (width 0.3) (layer "F.Cu") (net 1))
 (segment (start 90 60.75) (end 90 54.25) (width 0.3) (layer "F.Cu") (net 1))
 (segment (start 89.8 60.95) (end 90 60.75) (width 0.3) (layer "F.Cu") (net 1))
 (segment (start 91 61.75) (end 90 60.75) (width 0.3) (layer "F.Cu") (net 1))
 (segment (start 101.5875 61.75) (end 91 61.75) (width 0.3) (layer "F.Cu") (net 1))
 (segment (start 102 52.25) (end 105 55.25) (width 0.3) (layer "F.Cu") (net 39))
 (segment (start 84.75 71.487057) (end 84.75 61.909189) (width 0.3) (layer "F.Cu") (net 39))
 (segment (start 87.55 72.45) (end 85.712943 72.45) (width 0.3) (layer "F.Cu") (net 39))
 (segment (start 84.75 61.909189) (end 84.15 61.309189) (width 0.3) (layer "F.Cu") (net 39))
 (segment (start 85.712943 72.45) (end 84.75 71.487057) (width 0.3) (layer "F.Cu") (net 39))
 (segment (start 84.15 61.309189) (end 84.15 53.6) (width 0.3) (layer "F.Cu") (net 39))
 (segment (start 105 55.25) (end 105 57.3375) (width 0.3) (layer "F.Cu") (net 39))
 (segment (start 88.75 71.25) (end 87.55 72.45) (width 0.3) (layer "F.Cu") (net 39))
 (segment (start 84.15 53.6) (end 85.5 52.25) (width 0.3) (layer "F.Cu") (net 39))
 (segment (start 85.5 52.25) (end 102 52.25) (width 0.3) (layer "F.Cu") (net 39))
 (segment (start 88.75 68.71) (end 90.21 67.25) (width 0.3) (layer "F.Cu") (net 19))
 (segment (start 90.21 67.25) (end 92.5 67.25) (width 0.3) (layer "F.Cu") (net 19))
 (segment (start 92.5 67.25) (end 94.5 69.25) (width 0.3) (layer "F.Cu") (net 19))
 (segment (start 106.5 68) (end 106.5 65.6625) (width 0.3) (layer "F.Cu") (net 19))
 (segment (start 94.5 69.25) (end 105.25 69.25) (width 0.3) (layer "F.Cu") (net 19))
 (segment (start 105.25 69.25) (end 106.5 68) (width 0.3) (layer "F.Cu") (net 19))
 (segment (start 119.5 59.578709) (end 117.05 62.028709) (width 0.3) (layer "F.Cu") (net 37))
 (segment (start 117.548258 66.22) (end 118.25 66.22) (width 0.3) (layer "F.Cu") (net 37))
 (segment (start 116.811102 56) (end 119.5 58.688898) (width 0.3) (layer "F.Cu") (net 37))
 (segment (start 106.498959 56) (end 116.811102 56) (width 0.3) (layer "F.Cu") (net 37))
 (segment (start 117.05 62.028709) (end 117.05 65.02) (width 0.3) (layer "F.Cu") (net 37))
 (segment (start 115.459071 68.309187) (end 117.548258 66.22) (width 0.3) (layer "F.Cu") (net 37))
 (segment (start 106 57.3375) (end 106 56.498959) (width 0.3) (layer "F.Cu") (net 37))
 (segment (start 117.05 65.02) (end 118.25 66.22) (width 0.3) (layer "F.Cu") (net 37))
 (segment (start 119.5 58.688898) (end 119.5 59.578709) (width 0.3) (layer "F.Cu") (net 37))
 (segment (start 106 56.498959) (end 106.498959 56) (width 0.3) (layer "F.Cu") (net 37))
 (segment (start 112.270994 69.154794) (end 113.116601 68.309187) (width 0.3) (layer "F.Cu") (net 37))
 (segment (start 109.05 71.25) (end 111.145206 69.154794) (width 0.3) (layer "F.Cu") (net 37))
 (segment (start 113.116601 68.309187) (end 115.459071 68.309187) (width 0.3) (layer "F.Cu") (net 37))
 (segment (start 111.145206 69.154794) (end 112.270994 69.154794) (width 0.3) (layer "F.Cu") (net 37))
 (segment (start 119.614594 66.552463) (end 119.614594 65.044594) (width 0.3) (layer "F.Cu") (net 38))
 (segment (start 113.323707 68.809187) (end 115.910351 68.809187) (width 0.3) (layer "F.Cu") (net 38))
 (segment (start 112.4781 69.654794) (end 113.323707 68.809187) (width 0.3) (layer "F.Cu") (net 38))
 (segment (start 105.5 56.292558) (end 106.292558 55.5) (width 0.3) (layer "F.Cu") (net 38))
 (segment (start 119.614594 65.044594) (end 118.25 63.68) (width 0.3) (layer "F.Cu") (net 38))
 (segment (start 115.910351 68.809187) (end 117.299538 67.42) (width 0.3) (layer "F.Cu") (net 38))
 (segment (start 109.716423 72.45) (end 110.39 71.776423) (width 0.3) (layer "F.Cu") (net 38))
 (segment (start 110.39 71.776423) (end 110.39 70.752943) (width 0.3) (layer "F.Cu") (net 38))
 (segment (start 118.747057 67.42) (end 119.614594 66.552463) (width 0.3) (layer "F.Cu") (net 38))
 (segment (start 110.39 70.752943) (end 111.488149 69.654794) (width 0.3) (layer "F.Cu") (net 38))
 (segment (start 117.299538 67.42) (end 118.747057 67.42) (width 0.3) (layer "F.Cu") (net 38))
 (segment (start 111.488149 69.654794) (end 112.4781 69.654794) (width 0.3) (layer "F.Cu") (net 38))
 (segment (start 106.51 71.25) (end 107.71 72.45) (width 0.3) (layer "F.Cu") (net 38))
 (segment (start 107.71 72.45) (end 109.716423 72.45) (width 0.3) (layer "F.Cu") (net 38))
 (segment (start 106.51 71.25) (end 106.933668 71.25) (width 0.3) (layer "F.Cu") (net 38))
 (segment (start 120 61.93) (end 118.25 63.68) (width 0.3) (layer "F.Cu") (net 38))
 (segment (start 106.292558 55.5) (end 117.018208 55.5) (width 0.3) (layer "F.Cu") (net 38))
 (segment (start 105.5 57.3375) (end 105.5 56.292558) (width 0.3) (layer "F.Cu") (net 38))
 (segment (start 120 58.481792) (end 120 61.93) (width 0.3) (layer "F.Cu") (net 38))
 (segment (start 117.018208 55.5) (end 120 58.481792) (width 0.3) (layer "F.Cu") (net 38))
 (segment (start 110.257693 68.587154) (end 110.257693 64.595193) (width 0.3) (layer "F.Cu") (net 22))
 (segment (start 106.25 69.75) (end 106.68437 69.31563) (width 0.3) (layer "F.Cu") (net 22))
 (segment (start 106.68437 69.31563) (end 109.529217 69.31563) (width 0.3) (layer "F.Cu") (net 22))
 (segment (start 109.529217 69.31563) (end 110.257693 68.587154) (width 0.3) (layer "F.Cu") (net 22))
 (segment (start 97.85 69.75) (end 106.25 69.75) (width 0.3) (layer "F.Cu") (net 22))
 (segment (start 110.257693 64.595193) (end 109.9125 64.25) (width 0.3) (layer "F.Cu") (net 22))
 (segment (start 96.35 71.25) (end 97.85 69.75) (width 0.3) (layer "F.Cu") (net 22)))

